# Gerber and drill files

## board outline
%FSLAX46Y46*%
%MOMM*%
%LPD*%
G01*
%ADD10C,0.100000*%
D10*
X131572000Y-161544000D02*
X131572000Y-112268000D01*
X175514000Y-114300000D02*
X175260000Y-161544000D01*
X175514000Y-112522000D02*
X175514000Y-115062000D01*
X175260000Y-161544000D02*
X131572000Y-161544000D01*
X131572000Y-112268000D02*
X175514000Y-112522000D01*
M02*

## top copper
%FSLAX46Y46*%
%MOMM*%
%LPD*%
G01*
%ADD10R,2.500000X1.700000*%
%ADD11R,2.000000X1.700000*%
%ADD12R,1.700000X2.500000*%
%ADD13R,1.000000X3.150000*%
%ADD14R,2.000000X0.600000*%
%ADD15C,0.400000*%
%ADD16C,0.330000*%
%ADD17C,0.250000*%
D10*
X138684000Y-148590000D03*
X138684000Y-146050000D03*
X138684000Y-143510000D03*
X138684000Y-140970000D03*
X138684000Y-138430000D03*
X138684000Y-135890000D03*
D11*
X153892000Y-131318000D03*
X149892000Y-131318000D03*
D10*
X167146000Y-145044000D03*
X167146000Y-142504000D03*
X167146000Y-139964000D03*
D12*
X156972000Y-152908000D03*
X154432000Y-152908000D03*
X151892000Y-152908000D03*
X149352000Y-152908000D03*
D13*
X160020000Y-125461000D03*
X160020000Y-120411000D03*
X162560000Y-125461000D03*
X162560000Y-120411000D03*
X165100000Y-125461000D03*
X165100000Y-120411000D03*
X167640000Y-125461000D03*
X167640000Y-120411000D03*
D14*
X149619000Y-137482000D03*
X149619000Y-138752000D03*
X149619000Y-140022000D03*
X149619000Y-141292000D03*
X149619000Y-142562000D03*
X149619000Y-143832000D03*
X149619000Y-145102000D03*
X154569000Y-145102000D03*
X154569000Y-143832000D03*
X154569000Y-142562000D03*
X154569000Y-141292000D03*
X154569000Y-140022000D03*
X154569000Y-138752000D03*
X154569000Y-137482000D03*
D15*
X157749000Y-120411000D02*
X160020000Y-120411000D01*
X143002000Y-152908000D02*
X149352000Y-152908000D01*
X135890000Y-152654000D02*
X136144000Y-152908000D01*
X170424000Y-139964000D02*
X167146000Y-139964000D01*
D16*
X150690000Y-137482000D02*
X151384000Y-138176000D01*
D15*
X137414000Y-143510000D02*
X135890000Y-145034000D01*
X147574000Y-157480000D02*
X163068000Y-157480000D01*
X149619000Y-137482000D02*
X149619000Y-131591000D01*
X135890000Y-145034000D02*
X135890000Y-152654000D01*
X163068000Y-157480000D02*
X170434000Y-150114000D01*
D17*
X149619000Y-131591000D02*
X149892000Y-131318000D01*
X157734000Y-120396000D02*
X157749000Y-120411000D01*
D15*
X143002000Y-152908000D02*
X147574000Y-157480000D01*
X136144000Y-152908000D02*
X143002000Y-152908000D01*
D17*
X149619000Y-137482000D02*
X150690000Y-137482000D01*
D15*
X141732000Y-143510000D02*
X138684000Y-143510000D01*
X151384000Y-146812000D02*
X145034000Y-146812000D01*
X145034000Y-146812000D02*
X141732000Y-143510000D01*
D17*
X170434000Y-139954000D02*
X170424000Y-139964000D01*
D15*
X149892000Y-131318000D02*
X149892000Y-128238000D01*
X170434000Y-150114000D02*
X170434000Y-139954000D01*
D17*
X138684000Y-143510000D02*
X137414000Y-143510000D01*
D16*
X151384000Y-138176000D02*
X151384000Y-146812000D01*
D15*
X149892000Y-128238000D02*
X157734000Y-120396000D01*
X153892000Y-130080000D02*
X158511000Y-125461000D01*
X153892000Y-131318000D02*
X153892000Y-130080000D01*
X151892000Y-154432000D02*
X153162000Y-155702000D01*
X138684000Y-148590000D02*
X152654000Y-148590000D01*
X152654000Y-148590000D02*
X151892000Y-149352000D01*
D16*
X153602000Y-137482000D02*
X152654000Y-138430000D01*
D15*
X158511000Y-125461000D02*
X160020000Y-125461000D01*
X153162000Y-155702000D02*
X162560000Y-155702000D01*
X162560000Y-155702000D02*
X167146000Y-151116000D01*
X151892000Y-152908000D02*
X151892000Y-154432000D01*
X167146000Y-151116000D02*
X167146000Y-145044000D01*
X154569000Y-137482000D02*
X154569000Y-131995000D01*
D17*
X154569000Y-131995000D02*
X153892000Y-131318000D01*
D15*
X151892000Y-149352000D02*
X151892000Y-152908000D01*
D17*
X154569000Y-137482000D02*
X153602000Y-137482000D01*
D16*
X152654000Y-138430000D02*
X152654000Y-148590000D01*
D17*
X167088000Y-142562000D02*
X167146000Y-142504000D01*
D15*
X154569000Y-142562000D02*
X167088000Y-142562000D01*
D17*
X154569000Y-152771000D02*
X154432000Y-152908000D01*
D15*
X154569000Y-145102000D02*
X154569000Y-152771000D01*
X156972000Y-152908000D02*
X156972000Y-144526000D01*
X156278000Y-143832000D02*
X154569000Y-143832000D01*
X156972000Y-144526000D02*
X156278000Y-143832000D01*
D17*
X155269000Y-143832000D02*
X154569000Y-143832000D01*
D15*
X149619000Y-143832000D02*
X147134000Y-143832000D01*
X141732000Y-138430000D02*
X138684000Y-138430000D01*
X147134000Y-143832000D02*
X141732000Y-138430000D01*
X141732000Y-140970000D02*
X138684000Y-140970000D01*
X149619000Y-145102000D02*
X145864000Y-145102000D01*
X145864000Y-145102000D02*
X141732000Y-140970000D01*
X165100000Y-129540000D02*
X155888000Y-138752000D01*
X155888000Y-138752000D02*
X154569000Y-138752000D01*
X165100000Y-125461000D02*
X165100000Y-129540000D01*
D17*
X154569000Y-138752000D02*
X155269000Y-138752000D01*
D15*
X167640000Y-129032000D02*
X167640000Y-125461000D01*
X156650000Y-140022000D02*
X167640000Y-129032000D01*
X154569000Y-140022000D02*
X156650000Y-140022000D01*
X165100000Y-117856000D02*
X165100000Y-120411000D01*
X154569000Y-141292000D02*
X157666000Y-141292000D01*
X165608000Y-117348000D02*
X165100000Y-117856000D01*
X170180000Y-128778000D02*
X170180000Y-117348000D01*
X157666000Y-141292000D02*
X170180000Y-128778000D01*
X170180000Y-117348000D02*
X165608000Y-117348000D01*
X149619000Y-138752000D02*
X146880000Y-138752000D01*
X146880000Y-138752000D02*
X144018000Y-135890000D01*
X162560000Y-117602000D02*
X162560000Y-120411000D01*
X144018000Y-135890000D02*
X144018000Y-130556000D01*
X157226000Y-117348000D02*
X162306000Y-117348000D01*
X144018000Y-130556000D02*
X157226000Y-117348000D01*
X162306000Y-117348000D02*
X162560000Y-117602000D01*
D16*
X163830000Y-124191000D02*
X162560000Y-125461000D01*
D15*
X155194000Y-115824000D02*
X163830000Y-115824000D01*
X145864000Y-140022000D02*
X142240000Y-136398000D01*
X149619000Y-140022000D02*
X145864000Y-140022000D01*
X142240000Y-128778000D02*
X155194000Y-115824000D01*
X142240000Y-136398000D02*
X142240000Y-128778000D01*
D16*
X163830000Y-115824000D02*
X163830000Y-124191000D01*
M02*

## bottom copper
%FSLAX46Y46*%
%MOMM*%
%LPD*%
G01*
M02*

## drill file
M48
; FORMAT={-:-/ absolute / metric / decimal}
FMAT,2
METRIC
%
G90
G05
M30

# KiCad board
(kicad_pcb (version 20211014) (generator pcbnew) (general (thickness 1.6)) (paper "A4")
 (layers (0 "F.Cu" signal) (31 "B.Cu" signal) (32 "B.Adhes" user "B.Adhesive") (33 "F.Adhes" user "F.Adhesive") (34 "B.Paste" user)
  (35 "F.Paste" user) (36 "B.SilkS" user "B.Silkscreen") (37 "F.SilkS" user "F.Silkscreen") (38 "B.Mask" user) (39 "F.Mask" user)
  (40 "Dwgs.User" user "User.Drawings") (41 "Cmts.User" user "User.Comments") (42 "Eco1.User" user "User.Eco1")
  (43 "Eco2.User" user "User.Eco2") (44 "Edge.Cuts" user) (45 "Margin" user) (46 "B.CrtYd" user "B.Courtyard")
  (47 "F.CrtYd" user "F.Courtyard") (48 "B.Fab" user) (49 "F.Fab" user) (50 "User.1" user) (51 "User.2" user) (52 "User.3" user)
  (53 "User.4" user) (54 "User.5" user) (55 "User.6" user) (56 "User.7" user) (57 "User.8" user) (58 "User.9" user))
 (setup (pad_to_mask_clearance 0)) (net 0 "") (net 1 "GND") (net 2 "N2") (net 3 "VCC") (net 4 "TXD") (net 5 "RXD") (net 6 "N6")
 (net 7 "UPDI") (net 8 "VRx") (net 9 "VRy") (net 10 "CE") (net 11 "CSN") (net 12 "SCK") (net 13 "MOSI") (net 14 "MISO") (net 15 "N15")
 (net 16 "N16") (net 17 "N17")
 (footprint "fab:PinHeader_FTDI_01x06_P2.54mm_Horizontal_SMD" (layer "F.Cu") (at 138.684 148.59 180)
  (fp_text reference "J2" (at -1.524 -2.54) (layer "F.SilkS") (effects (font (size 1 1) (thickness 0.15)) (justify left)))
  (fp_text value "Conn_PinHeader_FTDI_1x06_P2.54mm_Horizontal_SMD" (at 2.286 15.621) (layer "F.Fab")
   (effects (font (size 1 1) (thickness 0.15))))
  (pad "1" smd rect locked (at 0 0 180) (size 2.5 1.7) (layers "F.Cu" "F.Paste" "F.Mask") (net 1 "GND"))
  (pad "2" smd rect locked (at 0 2.54 180) (size 2.5 1.7) (layers "F.Cu" "F.Paste" "F.Mask") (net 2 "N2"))
  (pad "3" smd rect locked (at 0 5.08 180) (size 2.5 1.7) (layers "F.Cu" "F.Paste" "F.Mask") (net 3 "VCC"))
  (pad "4" smd rect locked (at 0 7.62 180) (size 2.5 1.7) (layers "F.Cu" "F.Paste" "F.Mask") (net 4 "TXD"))
  (pad "5" smd rect locked (at 0 10.16 180) (size 2.5 1.7) (layers "F.Cu" "F.Paste" "F.Mask") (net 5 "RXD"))
  (pad "6" smd rect locked (at 0 12.7 180) (size 2.5 1.7) (layers "F.Cu" "F.Paste" "F.Mask") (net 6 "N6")))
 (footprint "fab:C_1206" (layer "F.Cu") (at 151.892 131.318 180)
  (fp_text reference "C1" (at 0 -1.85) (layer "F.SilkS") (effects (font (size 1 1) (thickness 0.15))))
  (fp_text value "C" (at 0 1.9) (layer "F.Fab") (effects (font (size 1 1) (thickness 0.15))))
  (pad "1" smd rect locked (at -2 0 180) (size 2 1.7) (layers "F.Cu" "F.Paste" "F.Mask") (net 1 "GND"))
  (pad "2" smd rect locked (at 2 0 180) (size 2 1.7) (layers "F.Cu" "F.Paste" "F.Mask") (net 3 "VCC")))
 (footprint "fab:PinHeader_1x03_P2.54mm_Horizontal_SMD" (layer "F.Cu") (at 167.146 145.044 180)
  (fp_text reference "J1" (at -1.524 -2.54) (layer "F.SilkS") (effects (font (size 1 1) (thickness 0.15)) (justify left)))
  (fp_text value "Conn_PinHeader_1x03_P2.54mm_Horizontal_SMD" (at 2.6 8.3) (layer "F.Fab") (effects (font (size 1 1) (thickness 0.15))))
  (pad "1" smd rect locked (at 0 0 180) (size 2.5 1.7) (layers "F.Cu" "F.Paste" "F.Mask") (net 1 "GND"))
  (pad "2" smd rect locked (at 0 2.54 180) (size 2.5 1.7) (layers "F.Cu" "F.Paste" "F.Mask") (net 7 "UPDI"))
  (pad "3" smd rect locked (at 0 5.08 180) (size 2.5 1.7) (layers "F.Cu" "F.Paste" "F.Mask") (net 3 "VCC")))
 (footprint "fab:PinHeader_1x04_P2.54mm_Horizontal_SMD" (layer "F.Cu") (at 156.972 152.908 -90)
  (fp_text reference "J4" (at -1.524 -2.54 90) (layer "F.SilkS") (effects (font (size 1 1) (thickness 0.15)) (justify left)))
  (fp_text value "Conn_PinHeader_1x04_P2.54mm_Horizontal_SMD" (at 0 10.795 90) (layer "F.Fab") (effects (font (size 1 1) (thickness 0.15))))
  (pad "1" smd rect locked (at 0 0 270) (size 2.5 1.7) (layers "F.Cu" "F.Paste" "F.Mask") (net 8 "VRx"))
  (pad "2" smd rect locked (at 0 2.54 270) (size 2.5 1.7) (layers "F.Cu" "F.Paste" "F.Mask") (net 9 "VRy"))
  (pad "3" smd rect locked (at 0 5.08 270) (size 2.5 1.7) (layers "F.Cu" "F.Paste" "F.Mask") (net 1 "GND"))
  (pad "4" smd rect locked (at 0 7.62 270) (size 2.5 1.7) (layers "F.Cu" "F.Paste" "F.Mask") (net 3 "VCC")))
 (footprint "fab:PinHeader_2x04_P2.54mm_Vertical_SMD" (layer "F.Cu") (at 163.83 122.936 90)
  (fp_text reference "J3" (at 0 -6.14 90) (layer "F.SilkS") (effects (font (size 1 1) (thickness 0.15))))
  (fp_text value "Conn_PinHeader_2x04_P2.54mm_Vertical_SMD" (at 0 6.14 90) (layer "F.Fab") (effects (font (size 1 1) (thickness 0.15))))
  (pad "1" smd rect locked (at -2.525 -3.81 90) (size 3.15 1) (layers "F.Cu" "F.Paste" "F.Mask") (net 1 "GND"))
  (pad "2" smd rect locked (at 2.525 -3.81 90) (size 3.15 1) (layers "F.Cu" "F.Paste" "F.Mask") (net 3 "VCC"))
  (pad "3" smd rect locked (at -2.525 -1.27 90) (size 3.15 1) (layers "F.Cu" "F.Paste" "F.Mask") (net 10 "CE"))
  (pad "4" smd rect locked (at 2.525 -1.27 90) (size 3.15 1) (layers "F.Cu" "F.Paste" "F.Mask") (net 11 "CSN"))
  (pad "5" smd rect locked (at -2.525 1.27 90) (size 3.15 1) (layers "F.Cu" "F.Paste" "F.Mask") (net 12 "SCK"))
  (pad "6" smd rect locked (at 2.525 1.27 90) (size 3.15 1) (layers "F.Cu" "F.Paste" "F.Mask") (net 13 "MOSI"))
  (pad "7" smd rect locked (at -2.525 3.81 90) (size 3.15 1) (layers "F.Cu" "F.Paste" "F.Mask") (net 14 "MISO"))
  (pad "8" smd rect locked (at 2.525 3.81 90) (size 3.15 1) (layers "F.Cu" "F.Paste" "F.Mask") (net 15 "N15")))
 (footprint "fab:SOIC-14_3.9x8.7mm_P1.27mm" (layer "F.Cu") (at 152.094 141.292)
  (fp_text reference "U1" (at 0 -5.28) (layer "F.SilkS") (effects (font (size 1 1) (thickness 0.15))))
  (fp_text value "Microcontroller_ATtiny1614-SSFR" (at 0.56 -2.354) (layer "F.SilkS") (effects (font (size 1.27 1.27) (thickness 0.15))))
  (pad "1" smd rect (at -2.475 -3.81) (size 2 0.6) (layers "F.Cu" "F.Paste" "F.Mask") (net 3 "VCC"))
  (pad "2" smd rect (at -2.475 -2.54) (size 2 0.6) (layers "F.Cu" "F.Paste" "F.Mask") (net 11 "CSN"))
  (pad "3" smd rect (at -2.475 -1.27) (size 2 0.6) (layers "F.Cu" "F.Paste" "F.Mask") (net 10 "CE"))
  (pad "4" smd rect (at -2.475 0) (size 2 0.6) (layers "F.Cu" "F.Paste" "F.Mask") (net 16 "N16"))
  (pad "5" smd rect (at -2.475 1.27) (size 2 0.6) (layers "F.Cu" "F.Paste" "F.Mask") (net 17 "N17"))
  (pad "6" smd rect (at -2.475 2.54) (size 2 0.6) (layers "F.Cu" "F.Paste" "F.Mask") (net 5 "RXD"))
  (pad "7" smd rect (at -2.475 3.81) (size 2 0.6) (layers "F.Cu" "F.Paste" "F.Mask") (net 4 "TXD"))
  (pad "8" smd rect (at 2.475 3.81) (size 2 0.6) (layers "F.Cu" "F.Paste" "F.Mask") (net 9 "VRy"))
  (pad "9" smd rect (at 2.475 2.54) (size 2 0.6) (layers "F.Cu" "F.Paste" "F.Mask") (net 8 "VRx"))
  (pad "10" smd rect (at 2.475 1.27) (size 2 0.6) (layers "F.Cu" "F.Paste" "F.Mask") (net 7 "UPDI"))
  (pad "11" smd rect (at 2.475 0) (size 2 0.6) (layers "F.Cu" "F.Paste" "F.Mask") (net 13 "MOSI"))
  (pad "12" smd rect (at 2.475 -1.27) (size 2 0.6) (layers "F.Cu" "F.Paste" "F.Mask") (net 14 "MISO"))
  (pad "13" smd rect (at 2.475 -2.54) (size 2 0.6) (layers "F.Cu" "F.Paste" "F.Mask") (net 12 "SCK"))
  (pad "14" smd rect (at 2.475 -3.81) (size 2 0.6) (layers "F.Cu" "F.Paste" "F.Mask") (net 1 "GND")))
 (gr_line (start 131.572 161.544) (end 131.572 112.268) (layer "Edge.Cuts") (width 0.1))
 (gr_line (start 175.514 114.3) (end 175.26 161.544) (layer "Edge.Cuts") (width 0.1))
 (gr_line (start 175.514 112.522) (end 175.514 115.062) (layer "Edge.Cuts") (width 0.1))
 (gr_line (start 175.26 161.544) (end 131.572 161.544) (layer "Edge.Cuts") (width 0.1))
 (gr_line (start 131.572 112.268) (end 175.514 112.522) (layer "Edge.Cuts") (width 0.1))
 (segment (start 157.749 120.411) (end 160.02 120.411) (width 0.4) (layer "F.Cu") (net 3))
 (segment (start 143.002 152.908) (end 149.352 152.908) (width 0.4) (layer "F.Cu") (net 3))
 (segment (start 135.89 152.654) (end 136.144 152.908) (width 0.4) (layer "F.Cu") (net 3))
 (segment (start 170.424 139.964) (end 167.146 139.964) (width 0.4) (layer "F.Cu") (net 3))
 (segment (start 150.69 137.482) (end 151.384 138.176) (width 0.33) (layer "F.Cu") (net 3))
 (segment (start 137.414 143.51) (end 135.89 145.034) (width 0.4) (layer "F.Cu") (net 3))
 (segment (start 147.574 157.48) (end 163.068 157.48) (width 0.4) (layer "F.Cu") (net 3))
 (segment (start 149.619 137.482) (end 149.619 131.591) (width 0.4) (layer "F.Cu") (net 3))
 (segment (start 135.89 145.034) (end 135.89 152.654) (width 0.4) (layer "F.Cu") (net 3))
 (segment (start 163.068 157.48) (end 170.434 150.114) (width 0.4) (layer "F.Cu") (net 3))
 (segment (start 149.619 131.591) (end 149.892 131.318) (width 0.25) (layer "F.Cu") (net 3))
 (segment (start 157.734 120.396) (end 157.749 120.411) (width 0.25) (layer "F.Cu") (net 3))
 (segment (start 143.002 152.908) (end 147.574 157.48) (width 0.4) (layer "F.Cu") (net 3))
 (segment (start 136.144 152.908) (end 143.002 152.908) (width 0.4) (layer "F.Cu") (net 3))
 (segment (start 149.619 137.482) (end 150.69 137.482) (width 0.25) (layer "F.Cu") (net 3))
 (segment (start 141.732 143.51) (end 138.684 143.51) (width 0.4) (layer "F.Cu") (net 3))
 (segment (start 151.384 146.812) (end 145.034 146.812) (width 0.4) (layer "F.Cu") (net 3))
 (segment (start 145.034 146.812) (end 141.732 143.51) (width 0.4) (layer "F.Cu") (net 3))
 (segment (start 170.434 139.954) (end 170.424 139.964) (width 0.25) (layer "F.Cu") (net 3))
 (segment (start 149.892 131.318) (end 149.892 128.238) (width 0.4) (layer "F.Cu") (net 3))
 (segment (start 170.434 150.114) (end 170.434 139.954) (width 0.4) (layer "F.Cu") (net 3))
 (segment (start 138.684 143.51) (end 137.414 143.51) (width 0.25) (layer "F.Cu") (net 3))
 (segment (start 151.384 138.176) (end 151.384 146.812) (width 0.33) (layer "F.Cu") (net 3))
 (segment (start 149.892 128.238) (end 157.734 120.396) (width 0.4) (layer "F.Cu") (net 3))
 (segment (start 153.892 130.08) (end 158.511 125.461) (width 0.4) (layer "F.Cu") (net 1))
 (segment (start 153.892 131.318) (end 153.892 130.08) (width 0.4) (layer "F.Cu") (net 1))
 (segment (start 151.892 154.432) (end 153.162 155.702) (width 0.4) (layer "F.Cu") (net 1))
 (segment (start 138.684 148.59) (end 152.654 148.59) (width 0.4) (layer "F.Cu") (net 1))
 (segment (start 152.654 148.59) (end 151.892 149.352) (width 0.4) (layer "F.Cu") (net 1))
 (segment (start 153.602 137.482) (end 152.654 138.43) (width 0.33) (layer "F.Cu") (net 1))
 (segment (start 158.511 125.461) (end 160.02 125.461) (width 0.4) (layer "F.Cu") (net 1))
 (segment (start 153.162 155.702) (end 162.56 155.702) (width 0.4) (layer "F.Cu") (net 1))
 (segment (start 162.56 155.702) (end 167.146 151.116) (width 0.4) (layer "F.Cu") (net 1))
 (segment (start 151.892 152.908) (end 151.892 154.432) (width 0.4) (layer "F.Cu") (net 1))
 (segment (start 167.146 151.116) (end 167.146 145.044) (width 0.4) (layer "F.Cu") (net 1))
 (segment (start 154.569 137.482) (end 154.569 131.995) (width 0.4) (layer "F.Cu") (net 1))
 (segment (start 154.569 131.995) (end 153.892 131.318) (width 0.25) (layer "F.Cu") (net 1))
 (segment (start 151.892 149.352) (end 151.892 152.908) (width 0.4) (layer "F.Cu") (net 1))
 (segment (start 154.569 137.482) (end 153.602 137.482) (width 0.25) (layer "F.Cu") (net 1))
 (segment (start 152.654 138.43) (end 152.654 148.59) (width 0.33) (layer "F.Cu") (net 1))
 (segment (start 167.088 142.562) (end 167.146 142.504) (width 0.25) (layer "F.Cu") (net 7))
 (segment (start 154.569 142.562) (end 167.088 142.562) (width 0.4) (layer "F.Cu") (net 7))
 (segment (start 154.569 152.771) (end 154.432 152.908) (width 0.25) (layer "F.Cu") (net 9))
 (segment (start 154.569 145.102) (end 154.569 152.771) (width 0.4) (layer "F.Cu") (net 9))
 (segment (start 156.972 152.908) (end 156.972 144.526) (width 0.4) (layer "F.Cu") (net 8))
 (segment (start 156.278 143.832) (end 154.569 143.832) (width 0.4) (layer "F.Cu") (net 8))
 (segment (start 156.972 144.526) (end 156.278 143.832) (width 0.4) (layer "F.Cu") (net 8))
 (segment (start 155.269 143.832) (end 154.569 143.832) (width 0.25) (layer "F.Cu") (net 8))
 (segment (start 149.619 143.832) (end 147.134 143.832) (width 0.4) (layer "F.Cu") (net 5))
 (segment (start 141.732 138.43) (end 138.684 138.43) (width 0.4) (layer "F.Cu") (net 5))
 (segment (start 147.134 143.832) (end 141.732 138.43) (width 0.4) (layer "F.Cu") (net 5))
 (segment (start 141.732 140.97) (end 138.684 140.97) (width 0.4) (layer "F.Cu") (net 4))
 (segment (start 149.619 145.102) (end 145.864 145.102) (width 0.4) (layer "F.Cu") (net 4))
 (segment (start 145.864 145.102) (end 141.732 140.97) (width 0.4) (layer "F.Cu") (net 4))
 (segment (start 165.1 129.54) (end 155.888 138.752) (width 0.4) (layer "F.Cu") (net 12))
 (segment (start 155.888 138.752) (end 154.569 138.752) (width 0.4) (layer "F.Cu") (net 12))
 (segment (start 165.1 125.461) (end 165.1 129.54) (width 0.4) (layer "F.Cu") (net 12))
 (segment (start 154.569 138.752) (end 155.269 138.752) (width 0.25) (layer "F.Cu") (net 12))
 (segment (start 167.64 129.032) (end 167.64 125.461) (width 0.4) (layer "F.Cu") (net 14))
 (segment (start 156.65 140.022) (end 167.64 129.032) (width 0.4) (layer "F.Cu") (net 14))
 (segment (start 154.569 140.022) (end 156.65 140.022) (width 0.4) (layer "F.Cu") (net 14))
 (segment (start 165.1 117.856) (end 165.1 120.411) (width 0.4) (layer "F.Cu") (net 13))
 (segment (start 154.569 141.292) (end 157.666 141.292) (width 0.4) (layer "F.Cu") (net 13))
 (segment (start 165.608 117.348) (end 165.1 117.856) (width 0.4) (layer "F.Cu") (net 13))
 (segment (start 170.18 128.778) (end 170.18 117.348) (width 0.4) (layer "F.Cu") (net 13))
 (segment (start 157.666 141.292) (end 170.18 128.778) (width 0.4) (layer "F.Cu") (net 13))
 (segment (start 170.18 117.348) (end 165.608 117.348) (width 0.4) (layer "F.Cu") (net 13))
 (segment (start 149.619 138.752) (end 146.88 138.752) (width 0.4) (layer "F.Cu") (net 11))
 (segment (start 146.88 138.752) (end 144.018 135.89) (width 0.4) (layer "F.Cu") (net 11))
 (segment (start 162.56 117.602) (end 162.56 120.411) (width 0.4) (layer "F.Cu") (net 11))
 (segment (start 144.018 135.89) (end 144.018 130.556) (width 0.4) (layer "F.Cu") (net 11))
 (segment (start 157.226 117.348) (end 162.306 117.348) (width 0.4) (layer "F.Cu") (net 11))
 (segment (start 144.018 130.556) (end 157.226 117.348) (width 0.4) (layer "F.Cu") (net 11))
 (segment (start 162.306 117.348) (end 162.56 117.602) (width 0.4) (layer "F.Cu") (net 11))
 (segment (start 163.83 124.191) (end 162.56 125.461) (width 0.33) (layer "F.Cu") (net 10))
 (segment (start 155.194 115.824) (end 163.83 115.824) (width 0.4) (layer "F.Cu") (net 10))
 (segment (start 145.864 140.022) (end 142.24 136.398) (width 0.4) (layer "F.Cu") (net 10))
 (segment (start 149.619 140.022) (end 145.864 140.022) (width 0.4) (layer "F.Cu") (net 10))
 (segment (start 142.24 128.778) (end 155.194 115.824) (width 0.4) (layer "F.Cu") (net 10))
 (segment (start 142.24 136.398) (end 142.24 128.778) (width 0.4) (layer "F.Cu") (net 10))
 (segment (start 163.83 115.824) (end 163.83 124.191) (width 0.33) (layer "F.Cu") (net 10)))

